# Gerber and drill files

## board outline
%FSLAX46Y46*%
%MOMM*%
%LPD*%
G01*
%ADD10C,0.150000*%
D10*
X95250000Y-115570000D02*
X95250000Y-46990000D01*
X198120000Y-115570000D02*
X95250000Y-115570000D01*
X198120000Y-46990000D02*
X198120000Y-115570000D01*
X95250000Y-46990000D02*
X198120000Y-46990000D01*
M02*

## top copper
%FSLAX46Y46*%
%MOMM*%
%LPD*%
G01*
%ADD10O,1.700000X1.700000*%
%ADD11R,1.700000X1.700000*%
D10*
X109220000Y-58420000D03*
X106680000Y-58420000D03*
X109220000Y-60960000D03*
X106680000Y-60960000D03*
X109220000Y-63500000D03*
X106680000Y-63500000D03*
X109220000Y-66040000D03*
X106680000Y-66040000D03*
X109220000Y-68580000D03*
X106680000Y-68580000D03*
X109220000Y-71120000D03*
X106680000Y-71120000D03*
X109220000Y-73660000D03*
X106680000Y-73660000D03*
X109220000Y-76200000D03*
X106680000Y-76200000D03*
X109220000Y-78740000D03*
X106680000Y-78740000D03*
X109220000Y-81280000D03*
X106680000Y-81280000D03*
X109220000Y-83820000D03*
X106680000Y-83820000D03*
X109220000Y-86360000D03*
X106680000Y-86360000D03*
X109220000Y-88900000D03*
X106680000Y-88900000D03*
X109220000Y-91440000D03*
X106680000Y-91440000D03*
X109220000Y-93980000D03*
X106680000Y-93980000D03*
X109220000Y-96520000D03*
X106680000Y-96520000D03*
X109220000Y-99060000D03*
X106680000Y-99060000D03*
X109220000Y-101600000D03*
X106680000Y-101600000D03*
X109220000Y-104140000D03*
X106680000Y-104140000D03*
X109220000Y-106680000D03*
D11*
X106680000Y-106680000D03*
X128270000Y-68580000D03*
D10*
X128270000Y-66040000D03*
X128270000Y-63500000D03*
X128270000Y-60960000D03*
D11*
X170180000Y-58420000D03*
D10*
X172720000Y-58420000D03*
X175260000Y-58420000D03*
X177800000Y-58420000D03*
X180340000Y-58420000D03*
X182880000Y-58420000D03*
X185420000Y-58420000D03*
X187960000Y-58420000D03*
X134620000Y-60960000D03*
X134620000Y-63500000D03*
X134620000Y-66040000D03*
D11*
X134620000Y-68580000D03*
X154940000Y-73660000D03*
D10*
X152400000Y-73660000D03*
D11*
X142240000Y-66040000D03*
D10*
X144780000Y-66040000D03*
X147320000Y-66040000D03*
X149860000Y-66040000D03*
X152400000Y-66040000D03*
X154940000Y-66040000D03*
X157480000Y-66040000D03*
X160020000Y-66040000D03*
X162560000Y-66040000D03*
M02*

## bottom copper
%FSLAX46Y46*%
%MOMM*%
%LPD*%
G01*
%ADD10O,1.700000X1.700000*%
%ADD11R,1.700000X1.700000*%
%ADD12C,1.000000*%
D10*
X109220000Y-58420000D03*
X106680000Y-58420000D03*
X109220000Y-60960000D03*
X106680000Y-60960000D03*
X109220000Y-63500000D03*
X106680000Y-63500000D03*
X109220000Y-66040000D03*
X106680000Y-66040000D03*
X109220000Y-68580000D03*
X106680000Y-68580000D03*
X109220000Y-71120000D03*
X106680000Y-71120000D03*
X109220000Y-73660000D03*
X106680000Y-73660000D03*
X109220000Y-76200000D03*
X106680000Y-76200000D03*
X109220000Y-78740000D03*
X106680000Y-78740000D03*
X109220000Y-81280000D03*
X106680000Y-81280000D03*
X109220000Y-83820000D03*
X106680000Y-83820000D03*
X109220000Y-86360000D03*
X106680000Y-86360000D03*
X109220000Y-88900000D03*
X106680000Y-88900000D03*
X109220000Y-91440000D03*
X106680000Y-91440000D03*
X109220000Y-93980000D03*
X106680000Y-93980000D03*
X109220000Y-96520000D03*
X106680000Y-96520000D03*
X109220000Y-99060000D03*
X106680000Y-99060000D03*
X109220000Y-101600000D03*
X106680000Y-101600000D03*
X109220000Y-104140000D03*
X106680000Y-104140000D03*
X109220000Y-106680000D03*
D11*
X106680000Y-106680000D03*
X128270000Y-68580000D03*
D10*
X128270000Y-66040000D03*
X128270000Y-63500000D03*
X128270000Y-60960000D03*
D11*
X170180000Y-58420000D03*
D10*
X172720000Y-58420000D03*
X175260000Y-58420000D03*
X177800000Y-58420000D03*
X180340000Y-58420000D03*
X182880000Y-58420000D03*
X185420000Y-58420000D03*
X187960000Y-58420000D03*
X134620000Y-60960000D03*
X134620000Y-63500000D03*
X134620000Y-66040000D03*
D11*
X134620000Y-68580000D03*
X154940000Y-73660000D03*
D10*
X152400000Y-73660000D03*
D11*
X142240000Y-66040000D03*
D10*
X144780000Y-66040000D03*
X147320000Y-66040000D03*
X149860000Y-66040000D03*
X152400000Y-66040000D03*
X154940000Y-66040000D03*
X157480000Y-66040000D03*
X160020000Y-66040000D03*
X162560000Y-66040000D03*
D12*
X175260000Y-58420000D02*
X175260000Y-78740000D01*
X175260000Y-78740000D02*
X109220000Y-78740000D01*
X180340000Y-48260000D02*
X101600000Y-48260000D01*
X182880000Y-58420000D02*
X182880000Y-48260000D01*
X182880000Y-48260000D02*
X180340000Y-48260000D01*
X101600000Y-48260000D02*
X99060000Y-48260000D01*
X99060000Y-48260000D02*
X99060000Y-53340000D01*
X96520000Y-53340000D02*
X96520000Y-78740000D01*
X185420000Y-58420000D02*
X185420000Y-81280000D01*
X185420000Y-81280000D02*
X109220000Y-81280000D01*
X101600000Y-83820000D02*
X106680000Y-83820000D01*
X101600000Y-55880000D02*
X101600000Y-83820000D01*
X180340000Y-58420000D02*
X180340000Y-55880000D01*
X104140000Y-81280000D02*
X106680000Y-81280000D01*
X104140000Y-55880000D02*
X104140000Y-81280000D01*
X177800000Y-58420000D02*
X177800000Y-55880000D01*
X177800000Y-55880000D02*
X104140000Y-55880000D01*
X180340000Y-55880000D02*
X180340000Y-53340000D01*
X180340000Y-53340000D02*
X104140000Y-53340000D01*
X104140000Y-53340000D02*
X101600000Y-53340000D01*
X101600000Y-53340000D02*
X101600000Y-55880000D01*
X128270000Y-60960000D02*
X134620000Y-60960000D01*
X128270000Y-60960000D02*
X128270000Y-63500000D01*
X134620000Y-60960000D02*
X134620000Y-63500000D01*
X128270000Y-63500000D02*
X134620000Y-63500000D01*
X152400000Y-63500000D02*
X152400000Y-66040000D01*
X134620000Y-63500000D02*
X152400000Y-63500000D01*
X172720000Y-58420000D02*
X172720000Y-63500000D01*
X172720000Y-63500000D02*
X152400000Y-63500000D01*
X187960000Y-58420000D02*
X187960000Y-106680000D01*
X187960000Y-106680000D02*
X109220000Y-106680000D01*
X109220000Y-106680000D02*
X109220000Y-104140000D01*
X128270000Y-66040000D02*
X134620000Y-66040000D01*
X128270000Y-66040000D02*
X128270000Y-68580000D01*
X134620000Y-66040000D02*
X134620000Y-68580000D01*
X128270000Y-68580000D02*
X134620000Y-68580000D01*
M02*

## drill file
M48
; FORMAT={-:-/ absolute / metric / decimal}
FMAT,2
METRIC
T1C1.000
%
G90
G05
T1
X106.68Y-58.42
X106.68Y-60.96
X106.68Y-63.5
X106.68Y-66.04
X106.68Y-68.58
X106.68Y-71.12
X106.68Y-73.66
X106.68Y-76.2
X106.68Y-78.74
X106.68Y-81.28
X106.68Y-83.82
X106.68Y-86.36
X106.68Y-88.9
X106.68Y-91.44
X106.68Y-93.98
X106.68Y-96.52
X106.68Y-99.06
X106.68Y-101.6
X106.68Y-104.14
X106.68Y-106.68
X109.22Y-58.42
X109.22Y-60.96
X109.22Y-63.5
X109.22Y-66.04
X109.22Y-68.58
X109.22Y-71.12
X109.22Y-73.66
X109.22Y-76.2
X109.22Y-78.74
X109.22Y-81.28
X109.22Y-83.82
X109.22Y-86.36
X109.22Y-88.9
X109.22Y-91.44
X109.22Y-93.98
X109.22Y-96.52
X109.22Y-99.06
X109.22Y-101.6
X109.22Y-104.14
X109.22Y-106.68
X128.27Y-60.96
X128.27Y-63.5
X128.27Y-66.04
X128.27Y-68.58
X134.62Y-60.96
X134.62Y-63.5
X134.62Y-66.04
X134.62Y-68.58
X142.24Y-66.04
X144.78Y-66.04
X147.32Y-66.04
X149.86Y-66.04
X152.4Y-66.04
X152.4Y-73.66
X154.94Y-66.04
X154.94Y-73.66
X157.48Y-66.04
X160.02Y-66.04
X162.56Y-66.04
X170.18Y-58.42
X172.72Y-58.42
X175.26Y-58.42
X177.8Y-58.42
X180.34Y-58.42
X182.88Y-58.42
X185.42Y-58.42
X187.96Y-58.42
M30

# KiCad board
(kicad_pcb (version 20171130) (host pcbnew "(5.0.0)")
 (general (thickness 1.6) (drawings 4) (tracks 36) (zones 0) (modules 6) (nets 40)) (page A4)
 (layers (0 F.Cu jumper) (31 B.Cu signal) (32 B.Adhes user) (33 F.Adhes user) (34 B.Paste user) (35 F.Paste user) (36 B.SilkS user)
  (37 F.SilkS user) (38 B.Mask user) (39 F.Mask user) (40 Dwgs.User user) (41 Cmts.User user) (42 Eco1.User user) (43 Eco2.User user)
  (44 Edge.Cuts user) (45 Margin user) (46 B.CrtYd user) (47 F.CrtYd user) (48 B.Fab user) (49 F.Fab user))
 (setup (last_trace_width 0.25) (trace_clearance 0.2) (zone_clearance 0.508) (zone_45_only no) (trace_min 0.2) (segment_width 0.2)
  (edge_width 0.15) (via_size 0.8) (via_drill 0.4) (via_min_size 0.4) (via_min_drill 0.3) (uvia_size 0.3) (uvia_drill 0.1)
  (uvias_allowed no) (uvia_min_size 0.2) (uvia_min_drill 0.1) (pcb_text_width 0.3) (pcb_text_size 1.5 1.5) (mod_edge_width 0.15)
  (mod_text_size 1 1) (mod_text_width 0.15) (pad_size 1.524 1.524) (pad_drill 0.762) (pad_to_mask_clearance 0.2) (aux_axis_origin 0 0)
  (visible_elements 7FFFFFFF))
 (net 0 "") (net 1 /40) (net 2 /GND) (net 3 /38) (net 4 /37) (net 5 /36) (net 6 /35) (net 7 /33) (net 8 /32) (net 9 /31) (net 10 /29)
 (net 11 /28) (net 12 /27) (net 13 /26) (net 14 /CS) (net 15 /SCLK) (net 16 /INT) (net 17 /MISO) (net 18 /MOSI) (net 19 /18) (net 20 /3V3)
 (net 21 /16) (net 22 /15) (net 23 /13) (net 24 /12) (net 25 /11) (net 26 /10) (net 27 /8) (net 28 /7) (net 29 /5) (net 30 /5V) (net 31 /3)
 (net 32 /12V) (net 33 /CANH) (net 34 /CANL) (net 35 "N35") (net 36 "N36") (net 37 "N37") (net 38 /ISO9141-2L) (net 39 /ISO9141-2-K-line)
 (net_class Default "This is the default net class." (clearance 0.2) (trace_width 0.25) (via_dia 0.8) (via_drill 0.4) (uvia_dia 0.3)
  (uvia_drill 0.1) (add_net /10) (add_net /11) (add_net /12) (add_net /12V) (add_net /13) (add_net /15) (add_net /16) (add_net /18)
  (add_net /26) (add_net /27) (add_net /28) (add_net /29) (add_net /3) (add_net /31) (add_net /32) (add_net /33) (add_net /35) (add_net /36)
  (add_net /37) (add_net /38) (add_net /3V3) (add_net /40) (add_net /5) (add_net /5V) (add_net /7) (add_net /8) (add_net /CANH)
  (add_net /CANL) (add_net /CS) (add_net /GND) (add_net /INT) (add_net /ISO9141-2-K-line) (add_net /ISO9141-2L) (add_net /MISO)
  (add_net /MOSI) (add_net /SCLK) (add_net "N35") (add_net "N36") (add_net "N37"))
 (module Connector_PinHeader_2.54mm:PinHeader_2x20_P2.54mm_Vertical (layer B.Cu) (at 106.68 106.68)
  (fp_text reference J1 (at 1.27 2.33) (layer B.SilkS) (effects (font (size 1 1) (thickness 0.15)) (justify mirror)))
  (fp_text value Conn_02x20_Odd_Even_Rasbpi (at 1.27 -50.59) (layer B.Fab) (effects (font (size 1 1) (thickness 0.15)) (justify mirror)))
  (pad 40 thru_hole oval (at 2.54 -48.26) (size 1.7 1.7) (drill 1) (layers *.Cu *.Mask) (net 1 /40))
  (pad 39 thru_hole oval (at 0 -48.26) (size 1.7 1.7) (drill 1) (layers *.Cu *.Mask) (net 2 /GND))
  (pad 38 thru_hole oval (at 2.54 -45.72) (size 1.7 1.7) (drill 1) (layers *.Cu *.Mask) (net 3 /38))
  (pad 37 thru_hole oval (at 0 -45.72) (size 1.7 1.7) (drill 1) (layers *.Cu *.Mask) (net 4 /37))
  (pad 36 thru_hole oval (at 2.54 -43.18) (size 1.7 1.7) (drill 1) (layers *.Cu *.Mask) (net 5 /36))
  (pad 35 thru_hole oval (at 0 -43.18) (size 1.7 1.7) (drill 1) (layers *.Cu *.Mask) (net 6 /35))
  (pad 34 thru_hole oval (at 2.54 -40.64) (size 1.7 1.7) (drill 1) (layers *.Cu *.Mask) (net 2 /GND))
  (pad 33 thru_hole oval (at 0 -40.64) (size 1.7 1.7) (drill 1) (layers *.Cu *.Mask) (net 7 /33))
  (pad 32 thru_hole oval (at 2.54 -38.1) (size 1.7 1.7) (drill 1) (layers *.Cu *.Mask) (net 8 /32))
  (pad 31 thru_hole oval (at 0 -38.1) (size 1.7 1.7) (drill 1) (layers *.Cu *.Mask) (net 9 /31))
  (pad 30 thru_hole oval (at 2.54 -35.56) (size 1.7 1.7) (drill 1) (layers *.Cu *.Mask) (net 2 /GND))
  (pad 29 thru_hole oval (at 0 -35.56) (size 1.7 1.7) (drill 1) (layers *.Cu *.Mask) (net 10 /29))
  (pad 28 thru_hole oval (at 2.54 -33.02) (size 1.7 1.7) (drill 1) (layers *.Cu *.Mask) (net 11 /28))
  (pad 27 thru_hole oval (at 0 -33.02) (size 1.7 1.7) (drill 1) (layers *.Cu *.Mask) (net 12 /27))
  (pad 26 thru_hole oval (at 2.54 -30.48) (size 1.7 1.7) (drill 1) (layers *.Cu *.Mask) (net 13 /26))
  (pad 25 thru_hole oval (at 0 -30.48) (size 1.7 1.7) (drill 1) (layers *.Cu *.Mask) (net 2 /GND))
  (pad 24 thru_hole oval (at 2.54 -27.94) (size 1.7 1.7) (drill 1) (layers *.Cu *.Mask) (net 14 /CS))
  (pad 23 thru_hole oval (at 0 -27.94) (size 1.7 1.7) (drill 1) (layers *.Cu *.Mask) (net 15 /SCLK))
  (pad 22 thru_hole oval (at 2.54 -25.4) (size 1.7 1.7) (drill 1) (layers *.Cu *.Mask) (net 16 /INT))
  (pad 21 thru_hole oval (at 0 -25.4) (size 1.7 1.7) (drill 1) (layers *.Cu *.Mask) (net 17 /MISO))
  (pad 20 thru_hole oval (at 2.54 -22.86) (size 1.7 1.7) (drill 1) (layers *.Cu *.Mask) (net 2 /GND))
  (pad 19 thru_hole oval (at 0 -22.86) (size 1.7 1.7) (drill 1) (layers *.Cu *.Mask) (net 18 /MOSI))
  (pad 18 thru_hole oval (at 2.54 -20.32) (size 1.7 1.7) (drill 1) (layers *.Cu *.Mask) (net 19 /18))
  (pad 17 thru_hole oval (at 0 -20.32) (size 1.7 1.7) (drill 1) (layers *.Cu *.Mask) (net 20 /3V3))
  (pad 16 thru_hole oval (at 2.54 -17.78) (size 1.7 1.7) (drill 1) (layers *.Cu *.Mask) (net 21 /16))
  (pad 15 thru_hole oval (at 0 -17.78) (size 1.7 1.7) (drill 1) (layers *.Cu *.Mask) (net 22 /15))
  (pad 14 thru_hole oval (at 2.54 -15.24) (size 1.7 1.7) (drill 1) (layers *.Cu *.Mask) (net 2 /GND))
  (pad 13 thru_hole oval (at 0 -15.24) (size 1.7 1.7) (drill 1) (layers *.Cu *.Mask) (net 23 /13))
  (pad 12 thru_hole oval (at 2.54 -12.7) (size 1.7 1.7) (drill 1) (layers *.Cu *.Mask) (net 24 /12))
  (pad 11 thru_hole oval (at 0 -12.7) (size 1.7 1.7) (drill 1) (layers *.Cu *.Mask) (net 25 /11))
  (pad 10 thru_hole oval (at 2.54 -10.16) (size 1.7 1.7) (drill 1) (layers *.Cu *.Mask) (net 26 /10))
  (pad 9 thru_hole oval (at 0 -10.16) (size 1.7 1.7) (drill 1) (layers *.Cu *.Mask) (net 2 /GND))
  (pad 8 thru_hole oval (at 2.54 -7.62) (size 1.7 1.7) (drill 1) (layers *.Cu *.Mask) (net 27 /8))
  (pad 7 thru_hole oval (at 0 -7.62) (size 1.7 1.7) (drill 1) (layers *.Cu *.Mask) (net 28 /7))
  (pad 6 thru_hole oval (at 2.54 -5.08) (size 1.7 1.7) (drill 1) (layers *.Cu *.Mask) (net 2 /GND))
  (pad 5 thru_hole oval (at 0 -5.08) (size 1.7 1.7) (drill 1) (layers *.Cu *.Mask) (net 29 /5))
  (pad 4 thru_hole oval (at 2.54 -2.54) (size 1.7 1.7) (drill 1) (layers *.Cu *.Mask) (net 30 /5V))
  (pad 3 thru_hole oval (at 0 -2.54) (size 1.7 1.7) (drill 1) (layers *.Cu *.Mask) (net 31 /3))
  (pad 2 thru_hole oval (at 2.54 0) (size 1.7 1.7) (drill 1) (layers *.Cu *.Mask) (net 30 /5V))
  (pad 1 thru_hole rect (at 0 0) (size 1.7 1.7) (drill 1) (layers *.Cu *.Mask) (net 20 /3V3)))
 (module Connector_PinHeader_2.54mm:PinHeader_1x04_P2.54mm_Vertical (layer F.Cu) (at 128.27 68.58 180)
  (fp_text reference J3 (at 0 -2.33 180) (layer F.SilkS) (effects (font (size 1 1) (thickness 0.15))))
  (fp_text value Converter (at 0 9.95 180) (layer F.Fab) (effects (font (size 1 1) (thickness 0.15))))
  (pad 1 thru_hole rect (at 0 0 180) (size 1.7 1.7) (drill 1) (layers *.Cu *.Mask) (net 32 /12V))
  (pad 2 thru_hole oval (at 0 2.54 180) (size 1.7 1.7) (drill 1) (layers *.Cu *.Mask) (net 32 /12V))
  (pad 3 thru_hole oval (at 0 5.08 180) (size 1.7 1.7) (drill 1) (layers *.Cu *.Mask) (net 2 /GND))
  (pad 4 thru_hole oval (at 0 7.62 180) (size 1.7 1.7) (drill 1) (layers *.Cu *.Mask) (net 2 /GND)))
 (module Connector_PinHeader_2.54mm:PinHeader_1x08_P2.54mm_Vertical (layer F.Cu) (at 170.18 58.42 90)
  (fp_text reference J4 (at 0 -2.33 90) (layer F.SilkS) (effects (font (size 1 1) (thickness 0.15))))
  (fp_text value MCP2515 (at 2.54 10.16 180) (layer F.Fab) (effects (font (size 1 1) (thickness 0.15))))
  (pad 1 thru_hole rect (at 0 0 90) (size 1.7 1.7) (drill 1) (layers *.Cu *.Mask) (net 20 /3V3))
  (pad 2 thru_hole oval (at 0 2.54 90) (size 1.7 1.7) (drill 1) (layers *.Cu *.Mask) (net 2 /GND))
  (pad 3 thru_hole oval (at 0 5.08 90) (size 1.7 1.7) (drill 1) (layers *.Cu *.Mask) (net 14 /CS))
  (pad 4 thru_hole oval (at 0 7.62 90) (size 1.7 1.7) (drill 1) (layers *.Cu *.Mask) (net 17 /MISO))
  (pad 5 thru_hole oval (at 0 10.16 90) (size 1.7 1.7) (drill 1) (layers *.Cu *.Mask) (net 18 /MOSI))
  (pad 6 thru_hole oval (at 0 12.7 90) (size 1.7 1.7) (drill 1) (layers *.Cu *.Mask) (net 15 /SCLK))
  (pad 7 thru_hole oval (at 0 15.24 90) (size 1.7 1.7) (drill 1) (layers *.Cu *.Mask) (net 16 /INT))
  (pad 8 thru_hole oval (at 0 17.78 90) (size 1.7 1.7) (drill 1) (layers *.Cu *.Mask) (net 30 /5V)))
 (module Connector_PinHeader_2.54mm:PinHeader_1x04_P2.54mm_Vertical (layer F.Cu) (at 134.62 68.58 180)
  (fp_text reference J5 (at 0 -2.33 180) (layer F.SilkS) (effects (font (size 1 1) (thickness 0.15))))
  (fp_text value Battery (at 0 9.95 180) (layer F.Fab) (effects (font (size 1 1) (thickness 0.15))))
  (pad 4 thru_hole oval (at 0 7.62 180) (size 1.7 1.7) (drill 1) (layers *.Cu *.Mask) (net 2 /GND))
  (pad 3 thru_hole oval (at 0 5.08 180) (size 1.7 1.7) (drill 1) (layers *.Cu *.Mask) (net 2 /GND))
  (pad 2 thru_hole oval (at 0 2.54 180) (size 1.7 1.7) (drill 1) (layers *.Cu *.Mask) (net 32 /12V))
  (pad 1 thru_hole rect (at 0 0 180) (size 1.7 1.7) (drill 1) (layers *.Cu *.Mask) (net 32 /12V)))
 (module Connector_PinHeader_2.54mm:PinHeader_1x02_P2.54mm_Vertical (layer F.Cu) (at 154.94 73.66 270)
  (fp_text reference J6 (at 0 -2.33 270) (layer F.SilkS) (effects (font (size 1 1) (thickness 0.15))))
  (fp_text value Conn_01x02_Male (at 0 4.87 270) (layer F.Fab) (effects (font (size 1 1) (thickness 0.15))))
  (pad 1 thru_hole rect (at 0 0 270) (size 1.7 1.7) (drill 1) (layers *.Cu *.Mask) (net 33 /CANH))
  (pad 2 thru_hole oval (at 0 2.54 270) (size 1.7 1.7) (drill 1) (layers *.Cu *.Mask) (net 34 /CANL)))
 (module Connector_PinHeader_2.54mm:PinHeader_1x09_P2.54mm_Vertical (layer F.Cu) (at 142.24 66.04 90)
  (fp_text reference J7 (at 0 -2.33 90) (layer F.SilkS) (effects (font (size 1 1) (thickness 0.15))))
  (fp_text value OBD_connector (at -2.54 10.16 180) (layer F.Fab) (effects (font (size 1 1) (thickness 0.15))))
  (pad 1 thru_hole rect (at 0 0 90) (size 1.7 1.7) (drill 1) (layers *.Cu *.Mask) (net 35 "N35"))
  (pad 2 thru_hole oval (at 0 2.54 90) (size 1.7 1.7) (drill 1) (layers *.Cu *.Mask) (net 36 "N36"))
  (pad 3 thru_hole oval (at 0 5.08 90) (size 1.7 1.7) (drill 1) (layers *.Cu *.Mask) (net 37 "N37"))
  (pad 4 thru_hole oval (at 0 7.62 90) (size 1.7 1.7) (drill 1) (layers *.Cu *.Mask) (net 34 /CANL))
  (pad 5 thru_hole oval (at 0 10.16 90) (size 1.7 1.7) (drill 1) (layers *.Cu *.Mask) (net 2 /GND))
  (pad 6 thru_hole oval (at 0 12.7 90) (size 1.7 1.7) (drill 1) (layers *.Cu *.Mask) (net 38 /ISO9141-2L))
  (pad 7 thru_hole oval (at 0 15.24 90) (size 1.7 1.7) (drill 1) (layers *.Cu *.Mask) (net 33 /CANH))
  (pad 8 thru_hole oval (at 0 17.78 90) (size 1.7 1.7) (drill 1) (layers *.Cu *.Mask) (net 32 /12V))
  (pad 9 thru_hole oval (at 0 20.32 90) (size 1.7 1.7) (drill 1) (layers *.Cu *.Mask) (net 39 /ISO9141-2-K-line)))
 (gr_line (start 95.25 115.57) (end 95.25 46.99) (layer Edge.Cuts) (width 0.15))
 (gr_line (start 198.12 115.57) (end 95.25 115.57) (layer Edge.Cuts) (width 0.15))
 (gr_line (start 198.12 46.99) (end 198.12 115.57) (layer Edge.Cuts) (width 0.15))
 (gr_line (start 95.25 46.99) (end 198.12 46.99) (layer Edge.Cuts) (width 0.15))
 (segment (start 175.26 58.42) (end 175.26 78.74) (width 1) (layer B.Cu) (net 14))
 (segment (start 175.26 78.74) (end 109.22 78.74) (width 1) (layer B.Cu) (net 14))
 (segment (start 180.34 48.26) (end 101.6 48.26) (width 1) (layer B.Cu) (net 15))
 (segment (start 182.88 58.42) (end 182.88 48.26) (width 1) (layer B.Cu) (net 15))
 (segment (start 182.88 48.26) (end 180.34 48.26) (width 1) (layer B.Cu) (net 15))
 (segment (start 101.6 48.26) (end 99.06 48.26) (width 1) (layer B.Cu) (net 15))
 (segment (start 99.06 48.26) (end 99.06 53.34) (width 1) (layer B.Cu) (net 15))
 (segment (start 96.52 53.34) (end 96.52 78.74) (width 1) (layer B.Cu) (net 15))
 (segment (start 185.42 58.42) (end 185.42 81.28) (width 1) (layer B.Cu) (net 16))
 (segment (start 185.42 81.28) (end 109.22 81.28) (width 1) (layer B.Cu) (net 16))
 (segment (start 101.6 83.82) (end 106.68 83.82) (width 1) (layer B.Cu) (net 18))
 (segment (start 101.6 55.88) (end 101.6 83.82) (width 1) (layer B.Cu) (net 18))
 (segment (start 180.34 58.42) (end 180.34 55.88) (width 1) (layer B.Cu) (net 18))
 (segment (start 104.14 81.28) (end 106.68 81.28) (width 1) (layer B.Cu) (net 17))
 (segment (start 104.14 55.88) (end 104.14 81.28) (width 1) (layer B.Cu) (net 17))
 (segment (start 177.8 58.42) (end 177.8 55.88) (width 1) (layer B.Cu) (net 17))
 (segment (start 177.8 55.88) (end 104.14 55.88) (width 1) (layer B.Cu) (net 17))
 (segment (start 180.34 55.88) (end 180.34 53.34) (width 1) (layer B.Cu) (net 18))
 (segment (start 180.34 53.34) (end 104.14 53.34) (width 1) (layer B.Cu) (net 18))
 (segment (start 104.14 53.34) (end 101.6 53.34) (width 1) (layer B.Cu) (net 18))
 (segment (start 101.6 53.34) (end 101.6 55.88) (width 1) (layer B.Cu) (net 18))
 (segment (start 128.27 60.96) (end 134.62 60.96) (width 1) (layer B.Cu) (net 2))
 (segment (start 128.27 60.96) (end 128.27 63.5) (width 1) (layer B.Cu) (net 2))
 (segment (start 134.62 60.96) (end 134.62 63.5) (width 1) (layer B.Cu) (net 2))
 (segment (start 128.27 63.5) (end 134.62 63.5) (width 1) (layer B.Cu) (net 2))
 (segment (start 152.4 63.5) (end 152.4 66.04) (width 1) (layer B.Cu) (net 2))
 (segment (start 134.62 63.5) (end 152.4 63.5) (width 1) (layer B.Cu) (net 2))
 (segment (start 172.72 58.42) (end 172.72 63.5) (width 1) (layer B.Cu) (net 2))
 (segment (start 172.72 63.5) (end 152.4 63.5) (width 1) (layer B.Cu) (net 2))
 (segment (start 187.96 58.42) (end 187.96 106.68) (width 1) (layer B.Cu) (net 30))
 (segment (start 187.96 106.68) (end 109.22 106.68) (width 1) (layer B.Cu) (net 30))
 (segment (start 109.22 106.68) (end 109.22 104.14) (width 1) (layer B.Cu) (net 30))
 (segment (start 128.27 66.04) (end 134.62 66.04) (width 1) (layer B.Cu) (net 32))
 (segment (start 128.27 66.04) (end 128.27 68.58) (width 1) (layer B.Cu) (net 32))
 (segment (start 134.62 66.04) (end 134.62 68.58) (width 1) (layer B.Cu) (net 32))
 (segment (start 128.27 68.58) (end 134.62 68.58) (width 1) (layer B.Cu) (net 32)))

